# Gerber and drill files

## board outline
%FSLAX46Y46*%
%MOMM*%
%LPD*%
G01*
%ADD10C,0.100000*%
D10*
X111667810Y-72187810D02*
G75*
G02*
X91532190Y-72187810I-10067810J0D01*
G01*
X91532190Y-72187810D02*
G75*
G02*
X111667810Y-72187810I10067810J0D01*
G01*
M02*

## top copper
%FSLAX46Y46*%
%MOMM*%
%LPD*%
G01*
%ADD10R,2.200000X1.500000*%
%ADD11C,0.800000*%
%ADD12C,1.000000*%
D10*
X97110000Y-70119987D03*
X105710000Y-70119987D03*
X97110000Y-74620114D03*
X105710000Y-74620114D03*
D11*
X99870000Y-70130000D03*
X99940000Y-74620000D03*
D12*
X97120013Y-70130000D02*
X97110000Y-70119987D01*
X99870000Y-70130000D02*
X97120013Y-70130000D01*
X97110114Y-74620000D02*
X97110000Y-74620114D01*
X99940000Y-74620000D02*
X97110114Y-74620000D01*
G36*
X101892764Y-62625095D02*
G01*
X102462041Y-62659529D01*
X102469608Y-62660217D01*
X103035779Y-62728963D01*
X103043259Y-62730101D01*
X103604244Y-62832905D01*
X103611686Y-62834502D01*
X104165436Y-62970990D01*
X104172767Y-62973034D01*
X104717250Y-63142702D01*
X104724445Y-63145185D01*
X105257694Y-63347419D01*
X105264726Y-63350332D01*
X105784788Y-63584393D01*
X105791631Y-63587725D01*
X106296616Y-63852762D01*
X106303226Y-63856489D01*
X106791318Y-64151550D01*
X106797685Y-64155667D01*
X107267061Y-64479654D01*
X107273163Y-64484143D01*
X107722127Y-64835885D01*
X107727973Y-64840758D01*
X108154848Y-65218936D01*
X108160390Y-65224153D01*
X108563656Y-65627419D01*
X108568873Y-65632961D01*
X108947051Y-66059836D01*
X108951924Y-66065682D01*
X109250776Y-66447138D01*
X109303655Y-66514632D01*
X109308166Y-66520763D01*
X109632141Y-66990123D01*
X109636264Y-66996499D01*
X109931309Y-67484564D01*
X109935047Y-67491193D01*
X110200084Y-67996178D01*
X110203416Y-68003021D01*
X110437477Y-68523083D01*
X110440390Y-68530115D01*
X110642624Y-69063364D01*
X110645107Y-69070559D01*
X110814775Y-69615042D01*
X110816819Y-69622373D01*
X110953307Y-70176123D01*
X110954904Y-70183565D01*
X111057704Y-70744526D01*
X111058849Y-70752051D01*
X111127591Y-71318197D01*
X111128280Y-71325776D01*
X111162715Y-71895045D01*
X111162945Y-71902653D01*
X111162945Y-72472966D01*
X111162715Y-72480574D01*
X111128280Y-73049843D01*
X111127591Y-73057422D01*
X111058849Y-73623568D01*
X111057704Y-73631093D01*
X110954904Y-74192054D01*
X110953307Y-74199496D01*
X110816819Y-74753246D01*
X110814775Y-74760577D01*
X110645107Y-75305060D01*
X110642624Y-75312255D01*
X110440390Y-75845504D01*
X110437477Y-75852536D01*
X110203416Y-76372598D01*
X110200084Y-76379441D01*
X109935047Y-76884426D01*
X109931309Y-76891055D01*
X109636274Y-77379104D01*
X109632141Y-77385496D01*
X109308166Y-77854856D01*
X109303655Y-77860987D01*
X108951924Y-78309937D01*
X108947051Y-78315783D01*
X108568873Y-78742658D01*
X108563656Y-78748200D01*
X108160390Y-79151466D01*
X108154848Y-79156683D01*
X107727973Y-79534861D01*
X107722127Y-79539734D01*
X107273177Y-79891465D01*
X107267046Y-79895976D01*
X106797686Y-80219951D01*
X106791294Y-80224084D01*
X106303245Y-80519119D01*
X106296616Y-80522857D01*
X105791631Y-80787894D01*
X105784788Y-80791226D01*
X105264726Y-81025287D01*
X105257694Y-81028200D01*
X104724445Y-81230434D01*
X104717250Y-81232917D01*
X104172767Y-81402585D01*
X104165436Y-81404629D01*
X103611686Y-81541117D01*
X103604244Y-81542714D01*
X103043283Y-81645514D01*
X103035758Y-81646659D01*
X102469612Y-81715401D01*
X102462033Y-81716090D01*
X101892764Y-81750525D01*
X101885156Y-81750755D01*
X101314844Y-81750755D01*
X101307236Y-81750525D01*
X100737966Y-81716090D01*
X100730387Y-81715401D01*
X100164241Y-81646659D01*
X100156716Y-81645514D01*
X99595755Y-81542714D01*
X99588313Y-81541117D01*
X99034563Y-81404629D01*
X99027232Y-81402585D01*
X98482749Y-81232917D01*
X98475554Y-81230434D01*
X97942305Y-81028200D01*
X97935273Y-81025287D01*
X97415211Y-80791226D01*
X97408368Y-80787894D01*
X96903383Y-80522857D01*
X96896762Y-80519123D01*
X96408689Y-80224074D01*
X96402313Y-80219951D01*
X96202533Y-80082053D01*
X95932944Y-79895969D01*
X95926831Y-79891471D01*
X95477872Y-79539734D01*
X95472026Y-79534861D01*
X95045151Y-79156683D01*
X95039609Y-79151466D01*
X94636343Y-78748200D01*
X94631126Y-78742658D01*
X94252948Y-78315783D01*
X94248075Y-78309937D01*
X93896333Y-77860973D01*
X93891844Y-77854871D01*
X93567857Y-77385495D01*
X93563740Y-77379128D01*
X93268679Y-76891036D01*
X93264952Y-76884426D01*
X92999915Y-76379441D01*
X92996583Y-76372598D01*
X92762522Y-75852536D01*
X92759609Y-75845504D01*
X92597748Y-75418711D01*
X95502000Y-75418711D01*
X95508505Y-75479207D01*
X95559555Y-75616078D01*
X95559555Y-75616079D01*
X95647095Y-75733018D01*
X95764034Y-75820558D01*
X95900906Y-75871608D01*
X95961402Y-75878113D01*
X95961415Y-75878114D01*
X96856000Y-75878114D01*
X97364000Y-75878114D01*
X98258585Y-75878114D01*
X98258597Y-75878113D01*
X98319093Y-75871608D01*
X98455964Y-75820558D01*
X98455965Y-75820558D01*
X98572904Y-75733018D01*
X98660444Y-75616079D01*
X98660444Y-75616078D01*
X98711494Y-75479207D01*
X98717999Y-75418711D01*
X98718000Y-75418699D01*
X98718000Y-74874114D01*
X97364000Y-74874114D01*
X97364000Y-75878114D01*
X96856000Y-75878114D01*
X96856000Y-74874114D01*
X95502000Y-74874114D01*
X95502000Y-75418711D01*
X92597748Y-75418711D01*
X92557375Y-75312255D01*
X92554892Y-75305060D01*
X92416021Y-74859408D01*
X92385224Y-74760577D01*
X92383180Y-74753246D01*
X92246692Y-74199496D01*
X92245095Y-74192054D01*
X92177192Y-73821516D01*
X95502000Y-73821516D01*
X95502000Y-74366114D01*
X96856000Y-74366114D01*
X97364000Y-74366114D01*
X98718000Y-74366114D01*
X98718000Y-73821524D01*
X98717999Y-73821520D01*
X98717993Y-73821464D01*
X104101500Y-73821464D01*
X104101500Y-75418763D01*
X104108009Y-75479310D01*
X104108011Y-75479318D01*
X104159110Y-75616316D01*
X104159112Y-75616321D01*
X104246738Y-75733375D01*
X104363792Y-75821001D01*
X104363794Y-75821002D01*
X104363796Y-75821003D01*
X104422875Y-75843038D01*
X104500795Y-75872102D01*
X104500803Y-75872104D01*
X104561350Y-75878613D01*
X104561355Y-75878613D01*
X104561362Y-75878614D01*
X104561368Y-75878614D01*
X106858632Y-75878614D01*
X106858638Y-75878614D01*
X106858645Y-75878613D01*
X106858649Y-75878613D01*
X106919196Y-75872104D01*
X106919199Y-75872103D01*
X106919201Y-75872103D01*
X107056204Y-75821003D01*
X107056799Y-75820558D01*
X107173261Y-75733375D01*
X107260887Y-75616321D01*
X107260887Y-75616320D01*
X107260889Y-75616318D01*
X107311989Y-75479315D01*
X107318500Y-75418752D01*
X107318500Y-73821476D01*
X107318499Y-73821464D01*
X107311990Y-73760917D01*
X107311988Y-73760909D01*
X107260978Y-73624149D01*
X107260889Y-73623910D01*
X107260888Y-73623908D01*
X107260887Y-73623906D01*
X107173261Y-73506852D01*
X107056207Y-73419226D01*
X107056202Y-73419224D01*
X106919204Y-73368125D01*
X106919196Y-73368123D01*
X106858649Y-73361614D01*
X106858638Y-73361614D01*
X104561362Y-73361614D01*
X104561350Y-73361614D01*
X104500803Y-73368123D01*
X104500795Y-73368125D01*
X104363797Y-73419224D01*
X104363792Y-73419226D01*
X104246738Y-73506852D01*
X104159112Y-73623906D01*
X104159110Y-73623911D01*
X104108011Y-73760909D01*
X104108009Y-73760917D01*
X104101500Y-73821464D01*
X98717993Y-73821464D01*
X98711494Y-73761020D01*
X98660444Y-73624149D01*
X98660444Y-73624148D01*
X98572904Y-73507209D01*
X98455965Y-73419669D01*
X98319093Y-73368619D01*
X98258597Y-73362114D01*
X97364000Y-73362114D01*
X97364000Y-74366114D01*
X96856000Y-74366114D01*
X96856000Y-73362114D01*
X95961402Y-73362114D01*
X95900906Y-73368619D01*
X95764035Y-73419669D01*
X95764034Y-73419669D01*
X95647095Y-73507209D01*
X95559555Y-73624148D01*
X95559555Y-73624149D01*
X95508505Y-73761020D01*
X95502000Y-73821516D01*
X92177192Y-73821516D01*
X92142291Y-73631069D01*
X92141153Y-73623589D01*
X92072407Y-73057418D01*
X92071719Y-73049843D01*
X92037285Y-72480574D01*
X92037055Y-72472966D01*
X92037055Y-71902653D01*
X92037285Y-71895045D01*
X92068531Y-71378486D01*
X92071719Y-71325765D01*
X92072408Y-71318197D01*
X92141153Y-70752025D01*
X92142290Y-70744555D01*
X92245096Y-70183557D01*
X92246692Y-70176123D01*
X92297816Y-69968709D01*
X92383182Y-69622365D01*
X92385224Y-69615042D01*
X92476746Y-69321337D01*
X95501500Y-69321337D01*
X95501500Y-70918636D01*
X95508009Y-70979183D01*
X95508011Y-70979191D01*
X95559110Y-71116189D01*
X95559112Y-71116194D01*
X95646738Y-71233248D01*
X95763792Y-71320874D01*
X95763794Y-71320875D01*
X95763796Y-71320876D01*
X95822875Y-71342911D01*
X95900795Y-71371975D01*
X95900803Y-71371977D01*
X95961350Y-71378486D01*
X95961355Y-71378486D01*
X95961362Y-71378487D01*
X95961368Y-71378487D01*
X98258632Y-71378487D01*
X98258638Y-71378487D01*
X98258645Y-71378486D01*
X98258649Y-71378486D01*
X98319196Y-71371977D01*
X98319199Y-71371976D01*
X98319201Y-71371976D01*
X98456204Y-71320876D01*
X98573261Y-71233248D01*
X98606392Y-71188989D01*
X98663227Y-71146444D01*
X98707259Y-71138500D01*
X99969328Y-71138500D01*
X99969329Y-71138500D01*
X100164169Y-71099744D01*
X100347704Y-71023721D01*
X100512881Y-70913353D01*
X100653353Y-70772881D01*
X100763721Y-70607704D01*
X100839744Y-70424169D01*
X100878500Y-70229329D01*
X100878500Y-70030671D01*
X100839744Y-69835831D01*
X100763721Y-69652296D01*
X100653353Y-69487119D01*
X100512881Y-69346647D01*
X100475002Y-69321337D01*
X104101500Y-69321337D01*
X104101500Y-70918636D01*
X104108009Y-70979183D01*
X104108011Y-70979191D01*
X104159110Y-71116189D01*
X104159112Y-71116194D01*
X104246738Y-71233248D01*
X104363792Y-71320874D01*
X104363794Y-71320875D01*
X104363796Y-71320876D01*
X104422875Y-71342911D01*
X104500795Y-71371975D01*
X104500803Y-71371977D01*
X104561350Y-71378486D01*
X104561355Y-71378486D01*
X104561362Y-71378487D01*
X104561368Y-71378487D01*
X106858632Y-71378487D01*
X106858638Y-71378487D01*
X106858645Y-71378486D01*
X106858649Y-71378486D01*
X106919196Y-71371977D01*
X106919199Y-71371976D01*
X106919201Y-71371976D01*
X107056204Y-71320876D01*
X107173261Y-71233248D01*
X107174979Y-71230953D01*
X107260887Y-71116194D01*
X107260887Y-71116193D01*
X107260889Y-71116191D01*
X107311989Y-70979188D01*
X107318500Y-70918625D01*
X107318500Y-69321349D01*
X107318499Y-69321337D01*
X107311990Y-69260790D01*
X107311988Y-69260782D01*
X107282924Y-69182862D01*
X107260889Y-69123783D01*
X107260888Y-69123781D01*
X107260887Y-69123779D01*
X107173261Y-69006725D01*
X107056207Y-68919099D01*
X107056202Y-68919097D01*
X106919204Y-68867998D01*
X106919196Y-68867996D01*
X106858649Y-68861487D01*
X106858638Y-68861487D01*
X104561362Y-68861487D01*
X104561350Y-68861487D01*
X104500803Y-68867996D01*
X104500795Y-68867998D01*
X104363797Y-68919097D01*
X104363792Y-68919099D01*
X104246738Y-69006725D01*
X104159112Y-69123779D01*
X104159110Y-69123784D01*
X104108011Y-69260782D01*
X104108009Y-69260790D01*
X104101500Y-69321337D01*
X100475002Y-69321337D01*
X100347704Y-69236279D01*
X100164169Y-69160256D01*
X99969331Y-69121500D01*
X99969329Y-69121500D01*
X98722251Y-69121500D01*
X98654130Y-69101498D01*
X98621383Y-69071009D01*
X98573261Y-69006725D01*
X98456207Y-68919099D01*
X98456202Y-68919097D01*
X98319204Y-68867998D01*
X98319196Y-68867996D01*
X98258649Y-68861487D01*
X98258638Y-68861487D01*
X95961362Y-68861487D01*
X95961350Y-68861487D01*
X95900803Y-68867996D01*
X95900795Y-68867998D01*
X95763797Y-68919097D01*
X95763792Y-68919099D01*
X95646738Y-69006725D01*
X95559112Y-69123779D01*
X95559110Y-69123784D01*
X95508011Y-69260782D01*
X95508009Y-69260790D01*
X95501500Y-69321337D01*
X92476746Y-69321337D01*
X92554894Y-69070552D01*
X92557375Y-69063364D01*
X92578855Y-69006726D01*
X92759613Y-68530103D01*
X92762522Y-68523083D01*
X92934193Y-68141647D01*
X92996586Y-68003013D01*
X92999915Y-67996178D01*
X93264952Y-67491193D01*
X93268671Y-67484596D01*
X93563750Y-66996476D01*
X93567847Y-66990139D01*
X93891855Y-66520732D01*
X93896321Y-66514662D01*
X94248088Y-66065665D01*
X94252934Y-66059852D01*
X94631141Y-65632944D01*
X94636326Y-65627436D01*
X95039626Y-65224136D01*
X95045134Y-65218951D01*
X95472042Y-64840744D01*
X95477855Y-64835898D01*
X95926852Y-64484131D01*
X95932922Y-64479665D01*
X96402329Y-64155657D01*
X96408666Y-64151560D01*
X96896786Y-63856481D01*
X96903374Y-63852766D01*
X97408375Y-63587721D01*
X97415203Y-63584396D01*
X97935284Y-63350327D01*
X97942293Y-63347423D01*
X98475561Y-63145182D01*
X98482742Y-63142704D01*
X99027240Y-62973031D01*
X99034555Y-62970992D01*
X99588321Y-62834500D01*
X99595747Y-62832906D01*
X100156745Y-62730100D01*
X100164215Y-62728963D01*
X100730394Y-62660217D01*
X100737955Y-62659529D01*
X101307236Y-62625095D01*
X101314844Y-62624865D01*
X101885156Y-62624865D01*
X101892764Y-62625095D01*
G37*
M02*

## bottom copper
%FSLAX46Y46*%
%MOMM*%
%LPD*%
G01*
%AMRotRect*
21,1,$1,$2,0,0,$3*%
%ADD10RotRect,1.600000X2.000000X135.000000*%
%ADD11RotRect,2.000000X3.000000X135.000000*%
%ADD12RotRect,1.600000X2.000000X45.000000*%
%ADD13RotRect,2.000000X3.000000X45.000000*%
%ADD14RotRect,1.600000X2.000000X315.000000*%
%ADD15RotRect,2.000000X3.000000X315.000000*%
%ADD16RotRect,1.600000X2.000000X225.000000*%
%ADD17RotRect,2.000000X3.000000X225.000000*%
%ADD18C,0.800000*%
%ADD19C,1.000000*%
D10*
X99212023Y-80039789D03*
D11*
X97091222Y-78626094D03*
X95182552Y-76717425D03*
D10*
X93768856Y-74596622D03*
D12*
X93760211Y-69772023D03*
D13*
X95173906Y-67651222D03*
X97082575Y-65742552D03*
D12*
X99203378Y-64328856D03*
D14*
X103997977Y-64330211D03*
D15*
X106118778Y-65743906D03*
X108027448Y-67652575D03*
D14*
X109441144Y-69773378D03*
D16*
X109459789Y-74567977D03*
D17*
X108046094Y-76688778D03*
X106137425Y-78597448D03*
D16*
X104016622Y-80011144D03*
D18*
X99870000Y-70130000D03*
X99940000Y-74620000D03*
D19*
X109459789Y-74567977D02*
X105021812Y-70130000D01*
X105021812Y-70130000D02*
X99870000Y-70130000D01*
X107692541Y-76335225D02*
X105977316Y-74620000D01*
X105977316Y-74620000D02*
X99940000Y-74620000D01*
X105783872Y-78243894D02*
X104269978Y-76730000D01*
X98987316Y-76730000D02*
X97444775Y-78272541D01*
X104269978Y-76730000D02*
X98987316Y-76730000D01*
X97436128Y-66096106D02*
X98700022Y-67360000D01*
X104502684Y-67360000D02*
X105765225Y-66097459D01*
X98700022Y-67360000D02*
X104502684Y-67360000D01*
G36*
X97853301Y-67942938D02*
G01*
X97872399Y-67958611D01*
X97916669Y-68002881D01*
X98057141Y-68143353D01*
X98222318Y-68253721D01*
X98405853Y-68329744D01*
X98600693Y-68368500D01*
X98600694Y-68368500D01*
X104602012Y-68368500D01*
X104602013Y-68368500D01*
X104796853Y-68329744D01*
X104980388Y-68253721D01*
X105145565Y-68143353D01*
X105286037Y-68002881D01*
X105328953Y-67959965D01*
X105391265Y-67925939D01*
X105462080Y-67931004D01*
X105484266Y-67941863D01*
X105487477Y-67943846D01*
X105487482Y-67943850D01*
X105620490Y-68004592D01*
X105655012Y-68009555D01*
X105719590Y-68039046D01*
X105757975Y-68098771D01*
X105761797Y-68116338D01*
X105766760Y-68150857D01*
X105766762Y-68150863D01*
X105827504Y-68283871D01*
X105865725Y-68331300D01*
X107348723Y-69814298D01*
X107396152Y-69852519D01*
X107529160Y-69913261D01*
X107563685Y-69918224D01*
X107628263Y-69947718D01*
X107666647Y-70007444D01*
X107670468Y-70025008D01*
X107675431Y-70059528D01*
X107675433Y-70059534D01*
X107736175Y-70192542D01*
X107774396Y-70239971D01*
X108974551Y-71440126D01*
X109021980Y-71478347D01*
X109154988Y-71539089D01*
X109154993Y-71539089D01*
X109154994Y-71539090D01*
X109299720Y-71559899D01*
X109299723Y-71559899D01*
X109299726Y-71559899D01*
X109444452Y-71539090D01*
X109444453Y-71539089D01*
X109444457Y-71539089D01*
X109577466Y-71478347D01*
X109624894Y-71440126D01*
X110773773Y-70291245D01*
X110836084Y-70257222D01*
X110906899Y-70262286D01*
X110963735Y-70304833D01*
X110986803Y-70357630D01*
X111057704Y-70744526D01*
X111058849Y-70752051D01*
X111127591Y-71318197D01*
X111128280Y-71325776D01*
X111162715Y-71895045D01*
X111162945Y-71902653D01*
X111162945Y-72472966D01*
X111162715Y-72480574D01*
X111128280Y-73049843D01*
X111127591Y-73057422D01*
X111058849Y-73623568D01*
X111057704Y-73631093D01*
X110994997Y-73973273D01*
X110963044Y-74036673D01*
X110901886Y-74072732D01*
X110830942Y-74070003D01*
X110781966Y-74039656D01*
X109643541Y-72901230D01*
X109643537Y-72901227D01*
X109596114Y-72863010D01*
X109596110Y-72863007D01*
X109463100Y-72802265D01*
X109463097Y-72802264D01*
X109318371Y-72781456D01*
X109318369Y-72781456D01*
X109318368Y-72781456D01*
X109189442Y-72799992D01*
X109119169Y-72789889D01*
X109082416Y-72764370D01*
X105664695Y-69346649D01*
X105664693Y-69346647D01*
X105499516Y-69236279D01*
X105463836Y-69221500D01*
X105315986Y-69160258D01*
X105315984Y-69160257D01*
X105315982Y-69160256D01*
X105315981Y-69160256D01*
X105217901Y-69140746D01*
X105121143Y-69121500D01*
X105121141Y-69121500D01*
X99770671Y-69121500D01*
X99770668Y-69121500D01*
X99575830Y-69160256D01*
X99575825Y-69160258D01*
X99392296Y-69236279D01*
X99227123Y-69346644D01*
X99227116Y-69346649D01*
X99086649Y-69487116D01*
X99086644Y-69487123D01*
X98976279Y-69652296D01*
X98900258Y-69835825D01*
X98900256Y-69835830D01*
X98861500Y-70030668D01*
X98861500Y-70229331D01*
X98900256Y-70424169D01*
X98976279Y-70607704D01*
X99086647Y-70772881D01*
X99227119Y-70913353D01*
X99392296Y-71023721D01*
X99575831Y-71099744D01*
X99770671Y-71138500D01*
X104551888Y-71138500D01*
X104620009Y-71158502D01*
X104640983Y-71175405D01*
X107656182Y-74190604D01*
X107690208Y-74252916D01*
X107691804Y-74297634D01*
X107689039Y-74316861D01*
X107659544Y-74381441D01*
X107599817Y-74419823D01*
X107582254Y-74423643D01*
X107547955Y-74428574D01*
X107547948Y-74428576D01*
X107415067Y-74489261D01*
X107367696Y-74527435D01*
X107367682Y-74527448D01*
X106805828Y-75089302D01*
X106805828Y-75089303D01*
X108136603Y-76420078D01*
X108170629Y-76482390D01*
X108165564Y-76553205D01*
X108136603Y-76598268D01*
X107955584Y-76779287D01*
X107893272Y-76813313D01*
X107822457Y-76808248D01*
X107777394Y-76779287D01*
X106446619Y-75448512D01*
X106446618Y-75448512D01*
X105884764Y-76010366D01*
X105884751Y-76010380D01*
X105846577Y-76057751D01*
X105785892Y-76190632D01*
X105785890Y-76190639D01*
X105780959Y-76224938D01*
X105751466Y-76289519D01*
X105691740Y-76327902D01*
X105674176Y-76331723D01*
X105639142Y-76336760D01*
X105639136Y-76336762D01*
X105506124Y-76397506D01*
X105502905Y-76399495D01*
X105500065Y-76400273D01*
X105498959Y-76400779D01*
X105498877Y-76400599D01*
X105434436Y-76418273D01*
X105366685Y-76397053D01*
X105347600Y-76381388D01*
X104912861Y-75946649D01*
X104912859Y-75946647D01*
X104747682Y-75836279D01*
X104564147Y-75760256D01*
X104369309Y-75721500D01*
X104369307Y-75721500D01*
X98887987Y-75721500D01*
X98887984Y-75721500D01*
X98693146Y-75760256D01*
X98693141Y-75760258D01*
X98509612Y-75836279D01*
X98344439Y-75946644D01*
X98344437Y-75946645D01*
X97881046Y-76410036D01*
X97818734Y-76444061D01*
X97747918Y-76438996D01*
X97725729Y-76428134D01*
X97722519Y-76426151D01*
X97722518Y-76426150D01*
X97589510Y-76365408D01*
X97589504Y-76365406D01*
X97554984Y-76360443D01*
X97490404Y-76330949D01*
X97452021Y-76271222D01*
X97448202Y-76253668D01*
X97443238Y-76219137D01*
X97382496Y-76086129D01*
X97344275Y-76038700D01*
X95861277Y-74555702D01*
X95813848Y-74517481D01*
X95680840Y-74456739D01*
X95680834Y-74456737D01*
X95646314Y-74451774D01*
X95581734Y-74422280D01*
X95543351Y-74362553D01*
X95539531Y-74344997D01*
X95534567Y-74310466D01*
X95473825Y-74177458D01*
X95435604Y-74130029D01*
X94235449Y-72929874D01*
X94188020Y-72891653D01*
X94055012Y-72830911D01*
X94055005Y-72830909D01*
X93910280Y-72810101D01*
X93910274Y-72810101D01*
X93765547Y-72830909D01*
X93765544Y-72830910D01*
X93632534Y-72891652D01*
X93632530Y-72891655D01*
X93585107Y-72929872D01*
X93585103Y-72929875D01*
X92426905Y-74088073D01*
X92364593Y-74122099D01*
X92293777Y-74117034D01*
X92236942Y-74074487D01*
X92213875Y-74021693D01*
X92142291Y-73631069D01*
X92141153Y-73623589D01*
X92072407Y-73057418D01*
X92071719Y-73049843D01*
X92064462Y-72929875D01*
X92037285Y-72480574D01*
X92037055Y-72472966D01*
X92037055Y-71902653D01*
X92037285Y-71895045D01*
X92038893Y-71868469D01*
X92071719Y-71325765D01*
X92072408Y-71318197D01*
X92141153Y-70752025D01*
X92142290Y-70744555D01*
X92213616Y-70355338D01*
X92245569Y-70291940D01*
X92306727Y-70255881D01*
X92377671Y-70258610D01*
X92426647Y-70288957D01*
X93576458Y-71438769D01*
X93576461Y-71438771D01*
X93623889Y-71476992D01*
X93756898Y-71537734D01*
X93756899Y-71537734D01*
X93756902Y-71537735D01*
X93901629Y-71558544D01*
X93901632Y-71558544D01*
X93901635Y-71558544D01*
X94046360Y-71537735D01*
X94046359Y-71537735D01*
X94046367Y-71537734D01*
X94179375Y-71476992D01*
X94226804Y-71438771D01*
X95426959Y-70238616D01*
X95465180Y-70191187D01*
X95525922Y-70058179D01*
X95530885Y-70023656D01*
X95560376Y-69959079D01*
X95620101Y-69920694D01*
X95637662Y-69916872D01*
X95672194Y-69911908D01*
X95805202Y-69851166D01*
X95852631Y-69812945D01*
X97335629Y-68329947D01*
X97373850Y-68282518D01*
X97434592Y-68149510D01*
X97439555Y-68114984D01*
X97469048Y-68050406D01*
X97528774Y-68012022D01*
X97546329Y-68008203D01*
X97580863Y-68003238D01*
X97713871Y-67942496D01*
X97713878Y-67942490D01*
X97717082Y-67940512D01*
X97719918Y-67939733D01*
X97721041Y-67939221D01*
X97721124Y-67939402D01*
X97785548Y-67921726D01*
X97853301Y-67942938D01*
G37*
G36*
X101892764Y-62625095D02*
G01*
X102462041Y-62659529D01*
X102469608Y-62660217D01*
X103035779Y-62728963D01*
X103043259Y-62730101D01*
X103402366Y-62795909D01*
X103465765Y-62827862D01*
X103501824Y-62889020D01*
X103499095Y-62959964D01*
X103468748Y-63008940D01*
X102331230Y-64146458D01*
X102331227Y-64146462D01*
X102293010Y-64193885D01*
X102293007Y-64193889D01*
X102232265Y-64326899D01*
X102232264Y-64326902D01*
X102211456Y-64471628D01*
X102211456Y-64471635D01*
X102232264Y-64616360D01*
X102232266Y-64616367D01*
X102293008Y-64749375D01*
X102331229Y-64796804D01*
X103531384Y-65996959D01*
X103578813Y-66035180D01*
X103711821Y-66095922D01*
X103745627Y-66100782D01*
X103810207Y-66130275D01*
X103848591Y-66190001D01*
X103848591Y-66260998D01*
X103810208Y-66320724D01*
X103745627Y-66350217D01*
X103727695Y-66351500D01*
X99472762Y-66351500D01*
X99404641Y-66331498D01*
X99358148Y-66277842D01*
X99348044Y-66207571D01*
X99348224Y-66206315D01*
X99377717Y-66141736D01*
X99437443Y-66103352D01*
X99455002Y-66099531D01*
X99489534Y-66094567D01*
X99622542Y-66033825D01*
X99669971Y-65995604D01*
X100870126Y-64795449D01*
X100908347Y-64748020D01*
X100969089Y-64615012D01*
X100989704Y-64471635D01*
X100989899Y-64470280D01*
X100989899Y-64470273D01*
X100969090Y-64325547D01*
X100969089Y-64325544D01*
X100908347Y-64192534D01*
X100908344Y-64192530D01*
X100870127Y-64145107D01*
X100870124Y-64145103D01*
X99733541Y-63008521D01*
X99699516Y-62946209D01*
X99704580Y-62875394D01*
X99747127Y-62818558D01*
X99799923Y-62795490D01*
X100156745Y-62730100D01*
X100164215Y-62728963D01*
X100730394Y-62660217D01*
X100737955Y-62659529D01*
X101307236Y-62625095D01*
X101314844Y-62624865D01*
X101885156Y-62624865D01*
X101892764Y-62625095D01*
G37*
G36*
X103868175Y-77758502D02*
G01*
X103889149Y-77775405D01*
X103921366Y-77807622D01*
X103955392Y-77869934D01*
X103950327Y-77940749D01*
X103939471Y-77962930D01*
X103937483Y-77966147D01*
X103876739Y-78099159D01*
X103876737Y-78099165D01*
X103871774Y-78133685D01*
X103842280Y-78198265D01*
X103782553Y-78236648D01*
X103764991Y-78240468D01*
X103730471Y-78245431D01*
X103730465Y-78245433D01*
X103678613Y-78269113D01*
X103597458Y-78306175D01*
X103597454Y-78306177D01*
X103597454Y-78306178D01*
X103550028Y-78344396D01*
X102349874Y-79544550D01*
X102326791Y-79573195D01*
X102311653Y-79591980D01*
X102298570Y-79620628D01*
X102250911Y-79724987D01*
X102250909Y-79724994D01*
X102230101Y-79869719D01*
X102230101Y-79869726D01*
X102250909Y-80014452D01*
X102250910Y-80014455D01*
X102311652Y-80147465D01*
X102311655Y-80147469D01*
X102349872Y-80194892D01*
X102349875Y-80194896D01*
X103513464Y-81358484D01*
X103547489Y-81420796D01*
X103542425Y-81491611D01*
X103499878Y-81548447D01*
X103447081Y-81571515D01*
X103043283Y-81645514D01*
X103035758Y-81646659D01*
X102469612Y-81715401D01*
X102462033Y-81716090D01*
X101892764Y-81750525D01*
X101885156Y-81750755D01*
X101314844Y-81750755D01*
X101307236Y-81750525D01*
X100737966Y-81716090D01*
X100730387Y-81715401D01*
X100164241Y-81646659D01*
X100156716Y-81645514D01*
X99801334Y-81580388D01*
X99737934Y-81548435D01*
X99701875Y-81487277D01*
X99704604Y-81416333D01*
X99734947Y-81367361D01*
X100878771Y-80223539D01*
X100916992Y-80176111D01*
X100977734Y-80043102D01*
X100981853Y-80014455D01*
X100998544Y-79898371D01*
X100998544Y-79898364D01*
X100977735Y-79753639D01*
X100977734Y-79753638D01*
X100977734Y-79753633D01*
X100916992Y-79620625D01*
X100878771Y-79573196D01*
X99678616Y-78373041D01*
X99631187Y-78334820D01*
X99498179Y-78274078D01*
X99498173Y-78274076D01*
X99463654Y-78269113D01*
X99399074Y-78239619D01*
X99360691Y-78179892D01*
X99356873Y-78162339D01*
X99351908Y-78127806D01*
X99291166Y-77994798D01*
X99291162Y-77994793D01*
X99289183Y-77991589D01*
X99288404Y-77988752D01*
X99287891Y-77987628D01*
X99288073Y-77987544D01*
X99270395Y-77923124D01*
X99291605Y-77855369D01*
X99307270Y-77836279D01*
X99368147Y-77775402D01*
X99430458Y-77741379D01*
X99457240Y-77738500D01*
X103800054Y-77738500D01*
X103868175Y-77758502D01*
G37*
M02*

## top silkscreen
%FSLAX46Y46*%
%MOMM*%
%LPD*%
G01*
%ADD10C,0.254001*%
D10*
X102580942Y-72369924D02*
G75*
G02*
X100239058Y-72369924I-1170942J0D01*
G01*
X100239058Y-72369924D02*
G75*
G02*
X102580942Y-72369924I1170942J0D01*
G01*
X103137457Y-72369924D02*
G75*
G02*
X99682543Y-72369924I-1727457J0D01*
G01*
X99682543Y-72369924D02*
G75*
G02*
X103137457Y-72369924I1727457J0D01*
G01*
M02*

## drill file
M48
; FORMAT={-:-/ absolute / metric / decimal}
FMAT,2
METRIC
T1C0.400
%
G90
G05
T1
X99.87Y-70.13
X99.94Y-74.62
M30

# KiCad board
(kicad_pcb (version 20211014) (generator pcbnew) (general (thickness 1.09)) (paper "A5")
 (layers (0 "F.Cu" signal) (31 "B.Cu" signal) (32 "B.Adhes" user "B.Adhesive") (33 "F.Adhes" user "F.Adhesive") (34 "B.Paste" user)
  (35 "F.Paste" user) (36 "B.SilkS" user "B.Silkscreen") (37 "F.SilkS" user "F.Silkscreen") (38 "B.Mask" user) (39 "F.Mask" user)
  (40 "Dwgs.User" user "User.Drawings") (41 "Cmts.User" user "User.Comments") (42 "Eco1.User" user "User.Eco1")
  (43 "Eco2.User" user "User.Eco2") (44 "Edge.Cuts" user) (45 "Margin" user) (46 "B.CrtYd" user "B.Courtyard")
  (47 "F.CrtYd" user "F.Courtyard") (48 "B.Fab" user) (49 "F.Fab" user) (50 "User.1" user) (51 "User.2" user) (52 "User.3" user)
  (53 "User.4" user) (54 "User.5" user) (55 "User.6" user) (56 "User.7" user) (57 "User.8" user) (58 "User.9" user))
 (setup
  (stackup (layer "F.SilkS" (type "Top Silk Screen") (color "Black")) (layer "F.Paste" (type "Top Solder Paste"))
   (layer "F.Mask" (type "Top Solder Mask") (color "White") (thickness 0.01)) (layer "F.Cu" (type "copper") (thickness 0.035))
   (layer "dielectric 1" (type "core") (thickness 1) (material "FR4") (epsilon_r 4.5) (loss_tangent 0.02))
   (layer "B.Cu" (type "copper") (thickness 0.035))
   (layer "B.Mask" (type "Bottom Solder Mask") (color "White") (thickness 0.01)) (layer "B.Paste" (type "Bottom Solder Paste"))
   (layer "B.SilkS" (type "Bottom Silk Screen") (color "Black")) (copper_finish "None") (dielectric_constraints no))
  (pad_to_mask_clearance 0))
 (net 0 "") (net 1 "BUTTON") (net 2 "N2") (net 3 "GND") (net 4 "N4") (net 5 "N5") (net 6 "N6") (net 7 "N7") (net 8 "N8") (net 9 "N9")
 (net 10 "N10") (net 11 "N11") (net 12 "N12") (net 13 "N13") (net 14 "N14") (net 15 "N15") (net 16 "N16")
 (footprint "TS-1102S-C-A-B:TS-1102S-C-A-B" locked (layer "F.Cu") (at 101.41 72.37)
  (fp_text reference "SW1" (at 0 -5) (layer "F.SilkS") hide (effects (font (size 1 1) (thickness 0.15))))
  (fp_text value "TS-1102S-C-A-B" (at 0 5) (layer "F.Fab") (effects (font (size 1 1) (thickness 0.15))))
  (fp_circle (center 0 -0.000076) (end 1.170942 -0.000076) (layer "F.SilkS") (width 0.254001) (fill none))
  (fp_circle (center 0 -0.000076) (end 1.727457 -0.000076) (layer "F.SilkS") (width 0.254001) (fill none))
  (pad "1" smd rect locked (at -4.3 -2.250013) (size 2.2 1.5) (layers "F.Cu" "F.Paste" "F.Mask") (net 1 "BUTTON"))
  (pad "2" smd rect locked (at 4.3 -2.250013) (size 2.2 1.5) (layers "F.Cu" "F.Paste" "F.Mask") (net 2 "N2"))
  (pad "3" smd rect locked (at -4.3 2.250114) (size 2.2 1.5) (layers "F.Cu" "F.Paste" "F.Mask") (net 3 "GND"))
  (pad "4" smd rect locked (at 4.3 2.250114) (size 2.2 1.5) (layers "F.Cu" "F.Paste" "F.Mask") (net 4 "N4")))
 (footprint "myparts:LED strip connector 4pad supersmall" (layer "B.Cu") (at 96.78 77.05 135)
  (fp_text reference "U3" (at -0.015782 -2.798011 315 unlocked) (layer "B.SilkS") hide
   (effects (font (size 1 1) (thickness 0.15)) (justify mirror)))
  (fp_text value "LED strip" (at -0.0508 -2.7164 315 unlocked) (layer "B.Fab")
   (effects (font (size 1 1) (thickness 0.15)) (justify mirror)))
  (pad "1" smd rect (at -3.8338 -0.3944 135) (size 1.6 2) (layers "B.Cu" "B.Mask") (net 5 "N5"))
  (pad "2" smd rect (at -1.334534 -0.8944 135) (size 2 3) (layers "B.Cu" "B.Mask") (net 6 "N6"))
  (pad "3" smd rect (at 1.364732 -0.8944 135) (size 2 3) (layers "B.Cu" "B.Mask") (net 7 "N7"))
  (pad "4" smd rect (at 3.864 -0.3944 135) (size 1.6 2) (layers "B.Cu" "B.Mask") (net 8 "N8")))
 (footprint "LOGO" (layer "B.Cu") (at 107.221884 72.021458 -135)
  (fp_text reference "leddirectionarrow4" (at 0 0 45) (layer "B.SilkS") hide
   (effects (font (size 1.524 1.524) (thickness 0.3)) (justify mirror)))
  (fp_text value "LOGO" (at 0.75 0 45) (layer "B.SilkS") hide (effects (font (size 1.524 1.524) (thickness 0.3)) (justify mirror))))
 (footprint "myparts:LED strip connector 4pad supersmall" (layer "B.Cu") (at 96.75 67.34 45)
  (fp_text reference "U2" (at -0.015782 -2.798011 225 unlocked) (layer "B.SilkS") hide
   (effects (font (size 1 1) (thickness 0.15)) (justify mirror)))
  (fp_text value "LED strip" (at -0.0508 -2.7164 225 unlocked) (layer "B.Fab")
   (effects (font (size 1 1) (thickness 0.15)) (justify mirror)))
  (pad "1" smd rect (at -3.8338 -0.3944 45) (size 1.6 2) (layers "B.Cu" "B.Mask") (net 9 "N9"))
  (pad "2" smd rect (at -1.334534 -0.8944 45) (size 2 3) (layers "B.Cu" "B.Mask") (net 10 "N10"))
  (pad "3" smd rect (at 1.364732 -0.8944 45) (size 2 3) (layers "B.Cu" "B.Mask") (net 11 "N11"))
  (pad "4" smd rect (at 3.864 -0.3944 45) (size 1.6 2) (layers "B.Cu" "B.Mask") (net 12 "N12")))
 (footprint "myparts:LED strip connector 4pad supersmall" (layer "B.Cu") (at 106.43 67.32 -45)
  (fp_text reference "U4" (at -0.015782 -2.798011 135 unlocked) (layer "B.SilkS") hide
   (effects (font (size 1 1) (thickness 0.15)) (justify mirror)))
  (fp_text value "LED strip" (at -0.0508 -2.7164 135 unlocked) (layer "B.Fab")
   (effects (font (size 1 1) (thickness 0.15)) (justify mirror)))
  (pad "1" smd rect (at -3.8338 -0.3944 315) (size 1.6 2) (layers "B.Cu" "B.Mask") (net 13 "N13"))
  (pad "2" smd rect (at -1.334534 -0.8944 315) (size 2 3) (layers "B.Cu" "B.Mask") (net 11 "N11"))
  (pad "3" smd rect (at 1.364732 -0.8944 315) (size 2 3) (layers "B.Cu" "B.Mask") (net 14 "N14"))
  (pad "4" smd rect (at 3.864 -0.3944 315) (size 1.6 2) (layers "B.Cu" "B.Mask") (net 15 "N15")))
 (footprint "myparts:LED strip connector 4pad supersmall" (layer "B.Cu") (at 106.47 77 -135)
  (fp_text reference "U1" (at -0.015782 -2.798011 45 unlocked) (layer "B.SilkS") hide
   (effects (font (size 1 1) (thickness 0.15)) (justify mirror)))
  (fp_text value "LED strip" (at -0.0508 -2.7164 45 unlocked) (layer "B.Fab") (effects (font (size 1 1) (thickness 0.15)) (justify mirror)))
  (pad "1" smd rect (at -3.8338 -0.3944 225) (size 1.6 2) (layers "B.Cu" "B.Mask") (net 1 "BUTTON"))
  (pad "2" smd rect (at -1.334534 -0.8944 225) (size 2 3) (layers "B.Cu" "B.Mask") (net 3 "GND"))
  (pad "3" smd rect (at 1.364732 -0.8944 225) (size 2 3) (layers "B.Cu" "B.Mask") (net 6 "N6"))
  (pad "4" smd rect (at 3.864 -0.3944 225) (size 1.6 2) (layers "B.Cu" "B.Mask") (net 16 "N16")))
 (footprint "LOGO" (layer "B.Cu") (at 96.228117 72.258542 45)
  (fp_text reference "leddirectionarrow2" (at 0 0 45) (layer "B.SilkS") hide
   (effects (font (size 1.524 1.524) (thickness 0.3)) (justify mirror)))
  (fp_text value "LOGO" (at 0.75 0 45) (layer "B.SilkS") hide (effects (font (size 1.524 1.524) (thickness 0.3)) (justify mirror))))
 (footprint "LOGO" (layer "B.Cu") (at 101.72 77.78 -45)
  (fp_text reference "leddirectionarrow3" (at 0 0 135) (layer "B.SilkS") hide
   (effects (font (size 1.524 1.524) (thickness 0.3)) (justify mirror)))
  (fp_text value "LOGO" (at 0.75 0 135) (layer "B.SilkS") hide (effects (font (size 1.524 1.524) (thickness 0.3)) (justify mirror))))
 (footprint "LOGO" (layer "B.Cu") (at 101.47 66.68 135)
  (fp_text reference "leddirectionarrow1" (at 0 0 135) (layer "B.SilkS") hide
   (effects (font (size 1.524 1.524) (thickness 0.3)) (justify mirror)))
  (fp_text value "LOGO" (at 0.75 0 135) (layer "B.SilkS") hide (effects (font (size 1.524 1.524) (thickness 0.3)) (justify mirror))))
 (gr_circle (center 101.6 72.18781) (end 111.62 73.16781) (layer "Edge.Cuts") (width 0.1) (fill none))
 (segment (start 97.120013 70.13) (end 97.11 70.119987) (width 1) (layer "F.Cu") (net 1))
 (segment (start 99.87 70.13) (end 97.120013 70.13) (width 1) (layer "F.Cu") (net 1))
 (via (at 99.87 70.13) (size 0.8) (drill 0.4) (layers "F.Cu" "B.Cu") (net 1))
 (segment (start 109.459789 74.567977) (end 105.021812 70.13) (width 1) (layer "B.Cu") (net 1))
 (segment (start 105.021812 70.13) (end 99.87 70.13) (width 1) (layer "B.Cu") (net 1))
 (segment (start 97.110114 74.62) (end 97.11 74.620114) (width 1) (layer "F.Cu") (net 3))
 (segment (start 99.94 74.62) (end 97.110114 74.62) (width 1) (layer "F.Cu") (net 3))
 (via (at 99.94 74.62) (size 0.8) (drill 0.4) (layers "F.Cu" "B.Cu") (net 3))
 (segment (start 107.692541 76.335225) (end 105.977316 74.62) (width 1) (layer "B.Cu") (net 3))
 (segment (start 105.977316 74.62) (end 99.94 74.62) (width 1) (layer "B.Cu") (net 3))
 (segment (start 105.783872 78.243894) (end 104.269978 76.73) (width 1) (layer "B.Cu") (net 6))
 (segment (start 98.987316 76.73) (end 97.444775 78.272541) (width 1) (layer "B.Cu") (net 6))
 (segment (start 104.269978 76.73) (end 98.987316 76.73) (width 1) (layer "B.Cu") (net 6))
 (segment (start 97.436128 66.096106) (end 98.700022 67.36) (width 1) (layer "B.Cu") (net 11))
 (segment (start 104.502684 67.36) (end 105.765225 66.097459) (width 1) (layer "B.Cu") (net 11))
 (segment (start 98.700022 67.36) (end 104.502684 67.36) (width 1) (layer "B.Cu") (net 11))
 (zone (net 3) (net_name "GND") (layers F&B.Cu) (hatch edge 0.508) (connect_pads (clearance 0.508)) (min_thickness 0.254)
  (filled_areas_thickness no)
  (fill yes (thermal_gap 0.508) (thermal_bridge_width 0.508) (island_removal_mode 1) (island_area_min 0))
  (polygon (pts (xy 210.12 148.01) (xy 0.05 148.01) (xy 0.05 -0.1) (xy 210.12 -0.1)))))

